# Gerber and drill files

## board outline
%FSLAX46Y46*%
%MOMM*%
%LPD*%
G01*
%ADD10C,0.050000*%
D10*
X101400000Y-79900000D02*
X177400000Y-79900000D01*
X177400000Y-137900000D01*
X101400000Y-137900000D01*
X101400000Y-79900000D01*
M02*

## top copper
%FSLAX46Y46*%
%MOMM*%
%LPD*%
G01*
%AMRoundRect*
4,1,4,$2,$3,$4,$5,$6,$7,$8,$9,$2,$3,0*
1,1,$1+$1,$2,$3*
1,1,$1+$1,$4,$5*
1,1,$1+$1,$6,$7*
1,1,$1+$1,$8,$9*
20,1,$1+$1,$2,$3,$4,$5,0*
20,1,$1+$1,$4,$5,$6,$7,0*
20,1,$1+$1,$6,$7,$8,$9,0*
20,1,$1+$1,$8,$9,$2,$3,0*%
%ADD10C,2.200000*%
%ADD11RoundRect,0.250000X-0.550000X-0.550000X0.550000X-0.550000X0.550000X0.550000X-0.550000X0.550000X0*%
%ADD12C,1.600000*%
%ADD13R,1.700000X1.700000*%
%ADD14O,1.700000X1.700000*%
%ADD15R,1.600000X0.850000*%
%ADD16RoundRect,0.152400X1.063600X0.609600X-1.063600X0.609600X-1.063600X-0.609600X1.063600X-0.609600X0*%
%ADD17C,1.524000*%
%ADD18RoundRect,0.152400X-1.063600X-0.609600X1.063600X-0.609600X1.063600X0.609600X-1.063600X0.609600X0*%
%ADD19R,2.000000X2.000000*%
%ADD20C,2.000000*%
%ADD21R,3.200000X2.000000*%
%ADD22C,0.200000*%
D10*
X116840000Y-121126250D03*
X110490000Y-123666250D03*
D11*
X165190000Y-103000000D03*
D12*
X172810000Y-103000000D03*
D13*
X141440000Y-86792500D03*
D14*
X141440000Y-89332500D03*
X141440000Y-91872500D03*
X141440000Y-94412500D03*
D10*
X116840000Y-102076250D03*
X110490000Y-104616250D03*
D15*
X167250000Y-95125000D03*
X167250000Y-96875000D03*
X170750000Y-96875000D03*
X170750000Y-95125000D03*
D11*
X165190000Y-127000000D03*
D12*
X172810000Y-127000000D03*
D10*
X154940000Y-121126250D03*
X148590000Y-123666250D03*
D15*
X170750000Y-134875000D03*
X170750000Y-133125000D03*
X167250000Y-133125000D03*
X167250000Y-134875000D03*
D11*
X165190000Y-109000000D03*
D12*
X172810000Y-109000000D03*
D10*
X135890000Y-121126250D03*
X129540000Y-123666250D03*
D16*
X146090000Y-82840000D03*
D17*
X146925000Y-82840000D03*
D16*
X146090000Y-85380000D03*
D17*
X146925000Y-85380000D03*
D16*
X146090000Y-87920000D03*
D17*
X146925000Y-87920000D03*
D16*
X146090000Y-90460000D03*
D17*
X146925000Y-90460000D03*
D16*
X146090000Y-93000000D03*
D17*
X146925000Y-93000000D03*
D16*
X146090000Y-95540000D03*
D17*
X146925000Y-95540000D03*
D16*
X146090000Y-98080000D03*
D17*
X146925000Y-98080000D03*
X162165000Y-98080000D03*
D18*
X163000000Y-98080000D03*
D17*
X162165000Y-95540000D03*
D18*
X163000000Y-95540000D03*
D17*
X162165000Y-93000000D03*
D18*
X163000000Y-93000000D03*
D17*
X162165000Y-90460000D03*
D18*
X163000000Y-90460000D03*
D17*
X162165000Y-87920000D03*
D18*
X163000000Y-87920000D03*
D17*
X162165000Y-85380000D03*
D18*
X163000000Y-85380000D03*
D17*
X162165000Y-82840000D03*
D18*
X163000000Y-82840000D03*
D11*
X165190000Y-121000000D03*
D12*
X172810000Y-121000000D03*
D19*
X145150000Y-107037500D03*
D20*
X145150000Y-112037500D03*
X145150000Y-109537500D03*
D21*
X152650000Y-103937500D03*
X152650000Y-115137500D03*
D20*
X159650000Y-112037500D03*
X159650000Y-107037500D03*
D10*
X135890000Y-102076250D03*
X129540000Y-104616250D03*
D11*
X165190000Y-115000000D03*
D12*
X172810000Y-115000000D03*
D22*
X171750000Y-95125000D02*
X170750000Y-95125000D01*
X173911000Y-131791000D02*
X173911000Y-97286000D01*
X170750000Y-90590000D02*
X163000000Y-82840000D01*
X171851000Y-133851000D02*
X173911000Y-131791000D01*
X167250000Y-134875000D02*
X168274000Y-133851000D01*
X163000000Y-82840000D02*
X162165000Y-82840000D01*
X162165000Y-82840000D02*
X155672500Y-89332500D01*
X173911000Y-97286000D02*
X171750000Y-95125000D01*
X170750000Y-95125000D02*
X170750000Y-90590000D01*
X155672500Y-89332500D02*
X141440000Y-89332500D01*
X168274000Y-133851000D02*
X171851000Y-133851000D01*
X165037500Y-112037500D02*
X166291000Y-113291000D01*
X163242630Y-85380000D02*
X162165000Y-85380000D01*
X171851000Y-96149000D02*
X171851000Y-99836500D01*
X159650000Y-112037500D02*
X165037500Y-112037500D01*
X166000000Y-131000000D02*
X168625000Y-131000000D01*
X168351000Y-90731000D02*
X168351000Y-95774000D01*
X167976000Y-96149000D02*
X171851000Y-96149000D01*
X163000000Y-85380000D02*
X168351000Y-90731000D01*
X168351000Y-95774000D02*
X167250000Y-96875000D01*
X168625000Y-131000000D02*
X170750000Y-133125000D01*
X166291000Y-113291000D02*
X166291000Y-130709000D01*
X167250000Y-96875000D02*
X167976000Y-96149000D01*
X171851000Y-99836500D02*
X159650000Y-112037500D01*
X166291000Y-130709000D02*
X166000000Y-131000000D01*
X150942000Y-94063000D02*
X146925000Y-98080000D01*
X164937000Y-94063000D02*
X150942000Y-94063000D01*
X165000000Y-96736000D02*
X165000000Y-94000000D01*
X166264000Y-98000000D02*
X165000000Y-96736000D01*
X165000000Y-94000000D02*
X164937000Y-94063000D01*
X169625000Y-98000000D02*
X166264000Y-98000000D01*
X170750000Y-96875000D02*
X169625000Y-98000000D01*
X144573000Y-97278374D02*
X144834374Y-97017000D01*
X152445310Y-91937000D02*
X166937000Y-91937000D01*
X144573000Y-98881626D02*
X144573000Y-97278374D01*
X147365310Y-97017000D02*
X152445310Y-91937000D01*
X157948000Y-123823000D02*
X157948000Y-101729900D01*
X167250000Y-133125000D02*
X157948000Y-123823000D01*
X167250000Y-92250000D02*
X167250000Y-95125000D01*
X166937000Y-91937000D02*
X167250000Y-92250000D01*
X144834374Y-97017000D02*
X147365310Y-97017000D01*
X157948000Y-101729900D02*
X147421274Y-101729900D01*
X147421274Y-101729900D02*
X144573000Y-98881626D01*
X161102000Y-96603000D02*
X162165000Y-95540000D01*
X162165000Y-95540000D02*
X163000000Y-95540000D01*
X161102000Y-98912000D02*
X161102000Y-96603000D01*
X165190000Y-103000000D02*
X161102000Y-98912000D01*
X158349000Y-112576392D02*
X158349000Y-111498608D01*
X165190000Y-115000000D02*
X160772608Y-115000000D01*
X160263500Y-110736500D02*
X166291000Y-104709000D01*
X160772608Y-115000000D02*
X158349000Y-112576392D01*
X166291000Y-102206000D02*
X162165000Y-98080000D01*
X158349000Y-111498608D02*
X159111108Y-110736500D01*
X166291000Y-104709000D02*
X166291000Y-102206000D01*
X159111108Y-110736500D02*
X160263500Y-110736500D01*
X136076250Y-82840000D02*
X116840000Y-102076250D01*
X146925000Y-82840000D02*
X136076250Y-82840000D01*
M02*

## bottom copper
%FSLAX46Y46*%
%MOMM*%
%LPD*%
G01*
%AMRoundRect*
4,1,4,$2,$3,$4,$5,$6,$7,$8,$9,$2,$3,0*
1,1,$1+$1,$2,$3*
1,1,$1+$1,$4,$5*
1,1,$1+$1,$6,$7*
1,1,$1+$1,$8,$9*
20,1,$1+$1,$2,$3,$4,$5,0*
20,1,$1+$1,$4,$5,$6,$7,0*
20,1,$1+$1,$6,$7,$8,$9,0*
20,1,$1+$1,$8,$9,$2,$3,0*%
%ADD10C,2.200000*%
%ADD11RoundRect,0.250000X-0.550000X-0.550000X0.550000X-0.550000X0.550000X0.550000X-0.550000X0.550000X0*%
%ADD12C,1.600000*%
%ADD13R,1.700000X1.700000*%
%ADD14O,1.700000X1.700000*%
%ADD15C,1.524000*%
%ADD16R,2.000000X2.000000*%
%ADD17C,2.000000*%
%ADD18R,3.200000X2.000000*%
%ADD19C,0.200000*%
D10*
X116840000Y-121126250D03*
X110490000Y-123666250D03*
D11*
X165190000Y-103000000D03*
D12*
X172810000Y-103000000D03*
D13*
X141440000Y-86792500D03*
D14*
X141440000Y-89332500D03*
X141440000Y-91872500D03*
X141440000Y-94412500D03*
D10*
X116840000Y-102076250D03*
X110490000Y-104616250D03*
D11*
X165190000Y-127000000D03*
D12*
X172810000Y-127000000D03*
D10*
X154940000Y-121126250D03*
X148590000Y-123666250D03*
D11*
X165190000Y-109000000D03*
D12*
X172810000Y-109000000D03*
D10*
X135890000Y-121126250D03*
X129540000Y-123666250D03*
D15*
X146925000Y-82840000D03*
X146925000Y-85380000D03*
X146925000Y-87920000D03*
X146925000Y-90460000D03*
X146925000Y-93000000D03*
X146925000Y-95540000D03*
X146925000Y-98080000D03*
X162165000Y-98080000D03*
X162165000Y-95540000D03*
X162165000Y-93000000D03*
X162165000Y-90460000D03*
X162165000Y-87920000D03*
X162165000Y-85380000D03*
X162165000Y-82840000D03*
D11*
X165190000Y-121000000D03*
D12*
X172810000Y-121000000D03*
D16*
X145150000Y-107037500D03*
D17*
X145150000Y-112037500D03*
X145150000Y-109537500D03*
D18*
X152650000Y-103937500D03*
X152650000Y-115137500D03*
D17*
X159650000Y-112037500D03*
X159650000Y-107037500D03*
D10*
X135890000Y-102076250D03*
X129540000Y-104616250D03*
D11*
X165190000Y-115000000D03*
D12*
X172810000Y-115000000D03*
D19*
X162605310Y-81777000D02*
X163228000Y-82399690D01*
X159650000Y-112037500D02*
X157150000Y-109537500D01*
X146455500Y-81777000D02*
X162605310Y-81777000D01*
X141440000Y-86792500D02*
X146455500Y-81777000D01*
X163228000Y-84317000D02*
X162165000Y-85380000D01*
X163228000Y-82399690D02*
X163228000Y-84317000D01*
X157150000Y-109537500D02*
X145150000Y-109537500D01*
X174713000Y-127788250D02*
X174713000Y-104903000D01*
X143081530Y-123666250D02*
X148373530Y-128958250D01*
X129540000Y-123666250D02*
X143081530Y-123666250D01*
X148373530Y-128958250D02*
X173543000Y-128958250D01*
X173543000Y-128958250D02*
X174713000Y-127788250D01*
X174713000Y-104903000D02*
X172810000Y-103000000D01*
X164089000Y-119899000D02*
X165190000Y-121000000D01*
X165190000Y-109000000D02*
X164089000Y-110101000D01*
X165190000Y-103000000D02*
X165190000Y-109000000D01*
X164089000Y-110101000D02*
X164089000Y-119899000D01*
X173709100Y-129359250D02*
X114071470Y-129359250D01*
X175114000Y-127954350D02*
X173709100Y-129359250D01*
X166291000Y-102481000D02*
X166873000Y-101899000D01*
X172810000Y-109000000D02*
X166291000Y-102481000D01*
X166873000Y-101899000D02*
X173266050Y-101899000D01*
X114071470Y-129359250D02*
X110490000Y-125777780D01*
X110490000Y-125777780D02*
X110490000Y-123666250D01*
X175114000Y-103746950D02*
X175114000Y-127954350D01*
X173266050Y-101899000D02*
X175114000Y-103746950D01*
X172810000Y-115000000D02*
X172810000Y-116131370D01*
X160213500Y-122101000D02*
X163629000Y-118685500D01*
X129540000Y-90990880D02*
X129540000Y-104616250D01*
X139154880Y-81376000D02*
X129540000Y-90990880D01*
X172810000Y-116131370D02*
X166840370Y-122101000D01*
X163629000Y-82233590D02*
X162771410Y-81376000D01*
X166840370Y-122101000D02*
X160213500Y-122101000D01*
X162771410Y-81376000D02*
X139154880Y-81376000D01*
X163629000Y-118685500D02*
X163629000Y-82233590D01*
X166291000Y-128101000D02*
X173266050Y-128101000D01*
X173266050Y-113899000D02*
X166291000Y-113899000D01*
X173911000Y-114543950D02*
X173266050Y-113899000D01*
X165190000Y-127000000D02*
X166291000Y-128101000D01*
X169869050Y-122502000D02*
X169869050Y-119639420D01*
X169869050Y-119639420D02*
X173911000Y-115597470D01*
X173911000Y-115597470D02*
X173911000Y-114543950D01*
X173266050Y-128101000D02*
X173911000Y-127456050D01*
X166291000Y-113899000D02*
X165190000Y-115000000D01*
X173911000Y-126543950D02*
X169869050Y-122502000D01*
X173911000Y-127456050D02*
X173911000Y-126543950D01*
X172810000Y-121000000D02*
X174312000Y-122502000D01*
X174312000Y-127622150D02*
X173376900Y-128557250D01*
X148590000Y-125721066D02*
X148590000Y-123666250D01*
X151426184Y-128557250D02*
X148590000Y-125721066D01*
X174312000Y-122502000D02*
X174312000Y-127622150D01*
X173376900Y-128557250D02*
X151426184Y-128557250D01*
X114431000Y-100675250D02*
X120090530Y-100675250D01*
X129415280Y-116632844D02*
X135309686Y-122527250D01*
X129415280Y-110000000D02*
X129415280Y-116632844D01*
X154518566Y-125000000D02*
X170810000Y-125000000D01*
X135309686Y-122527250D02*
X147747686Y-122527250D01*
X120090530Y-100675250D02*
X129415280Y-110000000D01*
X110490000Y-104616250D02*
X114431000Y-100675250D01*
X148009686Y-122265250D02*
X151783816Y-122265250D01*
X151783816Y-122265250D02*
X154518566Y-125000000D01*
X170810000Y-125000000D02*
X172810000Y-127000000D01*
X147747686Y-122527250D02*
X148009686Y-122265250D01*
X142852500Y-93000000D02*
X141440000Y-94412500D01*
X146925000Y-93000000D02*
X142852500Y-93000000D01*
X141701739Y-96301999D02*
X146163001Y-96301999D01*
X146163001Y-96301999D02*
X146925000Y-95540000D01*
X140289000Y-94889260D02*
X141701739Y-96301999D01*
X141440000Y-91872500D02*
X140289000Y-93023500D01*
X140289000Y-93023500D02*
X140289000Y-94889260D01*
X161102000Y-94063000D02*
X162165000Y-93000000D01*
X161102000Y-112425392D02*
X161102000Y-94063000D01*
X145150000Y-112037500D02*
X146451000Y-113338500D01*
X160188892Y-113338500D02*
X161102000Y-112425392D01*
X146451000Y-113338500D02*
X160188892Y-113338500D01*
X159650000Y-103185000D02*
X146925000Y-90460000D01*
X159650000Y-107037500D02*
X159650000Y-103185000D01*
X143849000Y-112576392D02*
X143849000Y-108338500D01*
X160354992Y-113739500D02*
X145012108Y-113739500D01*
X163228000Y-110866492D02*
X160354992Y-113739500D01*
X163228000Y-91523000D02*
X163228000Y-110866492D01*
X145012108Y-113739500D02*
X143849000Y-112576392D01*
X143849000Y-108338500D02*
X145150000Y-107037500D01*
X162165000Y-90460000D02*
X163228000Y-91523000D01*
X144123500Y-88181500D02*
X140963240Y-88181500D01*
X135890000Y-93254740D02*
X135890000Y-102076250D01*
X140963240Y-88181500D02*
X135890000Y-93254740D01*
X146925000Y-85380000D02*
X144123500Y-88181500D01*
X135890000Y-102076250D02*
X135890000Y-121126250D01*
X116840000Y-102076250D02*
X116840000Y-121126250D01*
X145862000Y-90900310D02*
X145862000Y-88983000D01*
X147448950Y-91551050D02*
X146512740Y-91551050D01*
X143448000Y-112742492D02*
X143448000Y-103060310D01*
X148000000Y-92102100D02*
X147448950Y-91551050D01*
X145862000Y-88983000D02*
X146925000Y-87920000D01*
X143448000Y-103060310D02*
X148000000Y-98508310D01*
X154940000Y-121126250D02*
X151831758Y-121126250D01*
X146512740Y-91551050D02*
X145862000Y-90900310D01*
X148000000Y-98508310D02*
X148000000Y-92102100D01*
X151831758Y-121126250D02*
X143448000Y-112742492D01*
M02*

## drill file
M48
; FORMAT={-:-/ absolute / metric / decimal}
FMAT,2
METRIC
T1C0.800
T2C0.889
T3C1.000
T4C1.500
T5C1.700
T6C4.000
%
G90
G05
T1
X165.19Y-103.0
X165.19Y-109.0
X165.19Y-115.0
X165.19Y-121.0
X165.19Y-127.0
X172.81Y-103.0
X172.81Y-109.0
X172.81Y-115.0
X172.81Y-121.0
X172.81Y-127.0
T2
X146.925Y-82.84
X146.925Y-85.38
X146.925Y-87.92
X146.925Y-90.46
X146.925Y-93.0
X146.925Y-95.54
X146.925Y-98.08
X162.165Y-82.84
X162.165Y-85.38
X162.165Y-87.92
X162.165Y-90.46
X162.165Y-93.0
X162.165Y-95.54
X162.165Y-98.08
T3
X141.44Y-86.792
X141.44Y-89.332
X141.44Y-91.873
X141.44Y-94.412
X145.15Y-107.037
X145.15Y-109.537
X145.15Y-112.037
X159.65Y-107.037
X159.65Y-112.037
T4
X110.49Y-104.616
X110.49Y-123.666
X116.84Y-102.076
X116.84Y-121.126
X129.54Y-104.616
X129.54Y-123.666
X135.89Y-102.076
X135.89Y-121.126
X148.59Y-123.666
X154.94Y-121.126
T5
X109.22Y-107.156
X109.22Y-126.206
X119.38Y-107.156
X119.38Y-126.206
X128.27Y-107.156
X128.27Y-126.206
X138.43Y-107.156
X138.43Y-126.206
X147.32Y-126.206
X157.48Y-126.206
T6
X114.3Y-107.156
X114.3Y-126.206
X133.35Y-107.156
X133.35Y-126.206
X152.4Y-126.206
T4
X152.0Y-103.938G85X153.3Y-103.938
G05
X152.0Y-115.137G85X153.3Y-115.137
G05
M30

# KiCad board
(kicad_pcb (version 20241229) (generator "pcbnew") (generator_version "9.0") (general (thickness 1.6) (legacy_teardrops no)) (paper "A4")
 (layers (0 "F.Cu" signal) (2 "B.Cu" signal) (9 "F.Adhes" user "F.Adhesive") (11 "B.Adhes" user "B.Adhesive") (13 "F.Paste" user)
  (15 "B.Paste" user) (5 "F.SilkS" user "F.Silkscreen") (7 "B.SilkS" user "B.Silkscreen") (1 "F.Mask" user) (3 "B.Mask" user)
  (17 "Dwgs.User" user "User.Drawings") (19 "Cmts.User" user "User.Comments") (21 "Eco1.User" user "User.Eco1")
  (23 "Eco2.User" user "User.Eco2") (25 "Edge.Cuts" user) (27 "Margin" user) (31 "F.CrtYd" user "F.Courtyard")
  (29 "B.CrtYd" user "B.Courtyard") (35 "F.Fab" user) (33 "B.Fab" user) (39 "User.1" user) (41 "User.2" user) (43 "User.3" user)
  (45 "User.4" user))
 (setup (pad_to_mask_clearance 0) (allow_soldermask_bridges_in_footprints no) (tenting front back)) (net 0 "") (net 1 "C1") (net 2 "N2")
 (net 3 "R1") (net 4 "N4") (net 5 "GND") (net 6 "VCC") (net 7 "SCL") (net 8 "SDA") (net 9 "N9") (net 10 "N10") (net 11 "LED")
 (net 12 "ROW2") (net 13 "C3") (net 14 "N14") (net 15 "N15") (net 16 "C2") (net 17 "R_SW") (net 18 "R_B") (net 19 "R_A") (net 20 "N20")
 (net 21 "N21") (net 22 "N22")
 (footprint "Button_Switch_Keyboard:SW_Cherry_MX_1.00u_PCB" (layer "F.Cu") (at 116.84 121.12625)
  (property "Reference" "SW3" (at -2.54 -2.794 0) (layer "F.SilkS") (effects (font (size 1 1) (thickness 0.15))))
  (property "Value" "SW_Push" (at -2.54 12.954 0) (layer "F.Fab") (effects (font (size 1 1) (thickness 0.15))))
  (pad "" np_thru_hole circle (at -7.62 5.08) (size 1.7 1.7) (drill 1.7) (layers "*.Cu" "*.Mask"))
  (pad "" np_thru_hole circle (at -2.54 5.08) (size 4 4) (drill 4) (layers "*.Cu" "*.Mask"))
  (pad "" np_thru_hole circle (at 2.54 5.08) (size 1.7 1.7) (drill 1.7) (layers "*.Cu" "*.Mask"))
  (pad "1" thru_hole circle (at 0 0) (size 2.2 2.2) (drill 1.5) (layers "*.Cu" "*.Mask") (remove_unused_layers no) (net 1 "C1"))
  (pad "2" thru_hole circle (at -6.35 2.54) (size 2.2 2.2) (drill 1.5) (layers "*.Cu" "*.Mask") (remove_unused_layers no) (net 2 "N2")))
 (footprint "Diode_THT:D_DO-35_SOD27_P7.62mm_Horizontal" (layer "F.Cu") (at 165.19 103)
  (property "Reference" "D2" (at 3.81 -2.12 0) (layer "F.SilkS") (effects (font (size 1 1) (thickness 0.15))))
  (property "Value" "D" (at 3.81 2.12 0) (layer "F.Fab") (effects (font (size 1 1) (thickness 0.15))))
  (pad "1" thru_hole roundrect (at 0 0) (size 1.6 1.6) (drill 0.8) (layers "*.Cu" "*.Mask") (remove_unused_layers no)
   (roundrect_rratio 0.15625) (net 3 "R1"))
  (pad "2" thru_hole circle (at 7.62 0) (size 1.6 1.6) (drill 0.8) (layers "*.Cu" "*.Mask") (remove_unused_layers no) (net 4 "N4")))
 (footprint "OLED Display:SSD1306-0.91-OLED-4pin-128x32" (layer "F.Cu") (at 104.94 84.6025)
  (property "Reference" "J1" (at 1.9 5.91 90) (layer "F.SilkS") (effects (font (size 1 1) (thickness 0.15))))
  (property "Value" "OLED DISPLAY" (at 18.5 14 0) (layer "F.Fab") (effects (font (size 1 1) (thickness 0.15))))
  (pad "1" thru_hole rect (at 36.5 2.19) (size 1.7 1.7) (drill 1) (layers "*.Cu" "*.Mask") (remove_unused_layers no) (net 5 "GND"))
  (pad "2" thru_hole oval (at 36.5 4.73) (size 1.7 1.7) (drill 1) (layers "*.Cu" "*.Mask") (remove_unused_layers no) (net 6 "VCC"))
  (pad "3" thru_hole oval (at 36.5 7.27) (size 1.7 1.7) (drill 1) (layers "*.Cu" "*.Mask") (remove_unused_layers no) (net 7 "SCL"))
  (pad "4" thru_hole oval (at 36.5 9.81) (size 1.7 1.7) (drill 1) (layers "*.Cu" "*.Mask") (remove_unused_layers no) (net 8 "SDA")))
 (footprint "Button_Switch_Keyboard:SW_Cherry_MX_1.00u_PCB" (layer "F.Cu") (at 116.84 102.07625)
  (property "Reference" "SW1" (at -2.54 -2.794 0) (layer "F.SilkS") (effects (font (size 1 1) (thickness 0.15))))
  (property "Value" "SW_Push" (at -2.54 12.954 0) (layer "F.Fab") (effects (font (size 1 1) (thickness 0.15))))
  (pad "" np_thru_hole circle (at -7.62 5.08) (size 1.7 1.7) (drill 1.7) (layers "*.Cu" "*.Mask"))
  (pad "" np_thru_hole circle (at -2.54 5.08) (size 4 4) (drill 4) (layers "*.Cu" "*.Mask"))
  (pad "" np_thru_hole circle (at 2.54 5.08) (size 1.7 1.7) (drill 1.7) (layers "*.Cu" "*.Mask"))
  (pad "1" thru_hole circle (at 0 0) (size 2.2 2.2) (drill 1.5) (layers "*.Cu" "*.Mask") (remove_unused_layers no) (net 1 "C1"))
  (pad "2" thru_hole circle (at -6.35 2.54) (size 2.2 2.2) (drill 1.5) (layers "*.Cu" "*.Mask") (remove_unused_layers no) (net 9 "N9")))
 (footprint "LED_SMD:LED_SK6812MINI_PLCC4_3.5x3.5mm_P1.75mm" (layer "F.Cu") (at 169 96)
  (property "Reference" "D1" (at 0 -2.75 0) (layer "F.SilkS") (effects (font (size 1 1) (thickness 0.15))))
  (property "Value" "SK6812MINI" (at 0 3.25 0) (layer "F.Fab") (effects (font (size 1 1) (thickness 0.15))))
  (pad "1" smd rect (at -1.75 -0.875) (size 1.6 0.85) (layers "F.Cu" "F.Mask" "F.Paste") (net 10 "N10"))
  (pad "2" smd rect (at -1.75 0.875) (size 1.6 0.85) (layers "F.Cu" "F.Mask" "F.Paste") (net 5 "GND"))
  (pad "3" smd rect (at 1.75 0.875) (size 1.6 0.85) (layers "F.Cu" "F.Mask" "F.Paste") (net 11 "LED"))
  (pad "4" smd rect (at 1.75 -0.875) (size 1.6 0.85) (layers "F.Cu" "F.Mask" "F.Paste") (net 6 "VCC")))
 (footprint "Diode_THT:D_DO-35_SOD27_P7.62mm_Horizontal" (layer "F.Cu") (at 165.19 127)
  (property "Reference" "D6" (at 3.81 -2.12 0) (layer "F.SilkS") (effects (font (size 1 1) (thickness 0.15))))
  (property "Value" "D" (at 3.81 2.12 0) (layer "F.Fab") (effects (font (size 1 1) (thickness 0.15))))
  (pad "1" thru_hole roundrect (at 0 0) (size 1.6 1.6) (drill 0.8) (layers "*.Cu" "*.Mask") (remove_unused_layers no)
   (roundrect_rratio 0.15625) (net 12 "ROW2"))
  (pad "2" thru_hole circle (at 7.62 0) (size 1.6 1.6) (drill 0.8) (layers "*.Cu" "*.Mask") (remove_unused_layers no) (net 9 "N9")))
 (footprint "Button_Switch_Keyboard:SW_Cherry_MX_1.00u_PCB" (layer "F.Cu") (at 154.94 121.12625)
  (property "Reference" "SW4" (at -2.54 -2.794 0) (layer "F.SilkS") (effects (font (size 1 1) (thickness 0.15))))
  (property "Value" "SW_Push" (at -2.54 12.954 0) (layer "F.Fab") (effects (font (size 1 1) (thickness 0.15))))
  (pad "" np_thru_hole circle (at -7.62 5.08) (size 1.7 1.7) (drill 1.7) (layers "*.Cu" "*.Mask"))
  (pad "" np_thru_hole circle (at -2.54 5.08) (size 4 4) (drill 4) (layers "*.Cu" "*.Mask"))
  (pad "" np_thru_hole circle (at 2.54 5.08) (size 1.7 1.7) (drill 1.7) (layers "*.Cu" "*.Mask"))
  (pad "1" thru_hole circle (at 0 0) (size 2.2 2.2) (drill 1.5) (layers "*.Cu" "*.Mask") (remove_unused_layers no) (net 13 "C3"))
  (pad "2" thru_hole circle (at -6.35 2.54) (size 2.2 2.2) (drill 1.5) (layers "*.Cu" "*.Mask") (remove_unused_layers no) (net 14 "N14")))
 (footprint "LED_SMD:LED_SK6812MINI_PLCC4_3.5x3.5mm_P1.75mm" (layer "F.Cu") (at 169 134 180)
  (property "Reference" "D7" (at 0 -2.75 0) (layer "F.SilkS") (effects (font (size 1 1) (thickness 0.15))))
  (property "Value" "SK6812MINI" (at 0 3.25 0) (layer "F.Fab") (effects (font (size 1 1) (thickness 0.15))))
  (pad "1" smd rect (at -1.75 -0.875 180) (size 1.6 0.85) (layers "F.Cu" "F.Mask" "F.Paste") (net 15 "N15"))
  (pad "2" smd rect (at -1.75 0.875 180) (size 1.6 0.85) (layers "F.Cu" "F.Mask" "F.Paste") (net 5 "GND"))
  (pad "3" smd rect (at 1.75 0.875 180) (size 1.6 0.85) (layers "F.Cu" "F.Mask" "F.Paste") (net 10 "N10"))
  (pad "4" smd rect (at 1.75 -0.875 180) (size 1.6 0.85) (layers "F.Cu" "F.Mask" "F.Paste") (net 6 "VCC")))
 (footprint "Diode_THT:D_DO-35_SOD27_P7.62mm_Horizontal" (layer "F.Cu") (at 165.19 109)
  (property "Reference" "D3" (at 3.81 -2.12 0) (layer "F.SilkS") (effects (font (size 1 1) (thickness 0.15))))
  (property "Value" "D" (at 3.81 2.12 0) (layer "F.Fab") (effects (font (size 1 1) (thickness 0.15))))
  (pad "1" thru_hole roundrect (at 0 0) (size 1.6 1.6) (drill 0.8) (layers "*.Cu" "*.Mask") (remove_unused_layers no)
   (roundrect_rratio 0.15625) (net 3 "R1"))
  (pad "2" thru_hole circle (at 7.62 0) (size 1.6 1.6) (drill 0.8) (layers "*.Cu" "*.Mask") (remove_unused_layers no) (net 2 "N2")))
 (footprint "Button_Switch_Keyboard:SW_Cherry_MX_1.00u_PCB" (layer "F.Cu") (at 135.89 121.12625)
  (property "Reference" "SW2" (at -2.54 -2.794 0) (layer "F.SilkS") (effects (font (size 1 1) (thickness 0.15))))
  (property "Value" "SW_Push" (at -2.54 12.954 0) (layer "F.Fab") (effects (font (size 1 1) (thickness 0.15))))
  (pad "" np_thru_hole circle (at -7.62 5.08) (size 1.7 1.7) (drill 1.7) (layers "*.Cu" "*.Mask"))
  (pad "" np_thru_hole circle (at -2.54 5.08) (size 4 4) (drill 4) (layers "*.Cu" "*.Mask"))
  (pad "" np_thru_hole circle (at 2.54 5.08) (size 1.7 1.7) (drill 1.7) (layers "*.Cu" "*.Mask"))
  (pad "1" thru_hole circle (at 0 0) (size 2.2 2.2) (drill 1.5) (layers "*.Cu" "*.Mask") (remove_unused_layers no) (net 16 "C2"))
  (pad "2" thru_hole circle (at -6.35 2.54) (size 2.2 2.2) (drill 1.5) (layers "*.Cu" "*.Mask") (remove_unused_layers no) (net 4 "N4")))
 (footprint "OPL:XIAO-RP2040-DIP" (layer "F.Cu") (at 154.545 90.46)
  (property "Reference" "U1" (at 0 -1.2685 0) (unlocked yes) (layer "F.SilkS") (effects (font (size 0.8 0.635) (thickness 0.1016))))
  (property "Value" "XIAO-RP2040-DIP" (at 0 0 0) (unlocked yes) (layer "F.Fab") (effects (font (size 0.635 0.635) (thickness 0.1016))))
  (pad "1" smd roundrect (at -8.455 -7.62 180) (size 2.432 1.524) (layers "F.Cu" "F.Mask") (roundrect_rratio 0.1) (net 1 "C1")
   (thermal_bridge_angle 45))
  (pad "1" thru_hole circle (at -7.62 -7.62 180) (size 1.524 1.524) (drill 0.889) (layers "*.Cu" "*.Mask") (remove_unused_layers no)
   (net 1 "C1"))
  (pad "2" smd roundrect (at -8.455 -5.08 180) (size 2.432 1.524) (layers "F.Cu" "F.Mask") (roundrect_rratio 0.1) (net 16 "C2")
   (thermal_bridge_angle 45))
  (pad "2" thru_hole circle (at -7.62 -5.08 180) (size 1.524 1.524) (drill 0.889) (layers "*.Cu" "*.Mask") (remove_unused_layers no)
   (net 16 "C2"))
  (pad "3" smd roundrect (at -8.455 -2.54 180) (size 2.432 1.524) (layers "F.Cu" "F.Mask") (roundrect_rratio 0.1) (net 13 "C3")
   (thermal_bridge_angle 45))
  (pad "3" thru_hole circle (at -7.62 -2.54 180) (size 1.524 1.524) (drill 0.889) (layers "*.Cu" "*.Mask") (remove_unused_layers no)
   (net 13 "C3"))
  (pad "4" smd roundrect (at -8.455 0 180) (size 2.432 1.524) (layers "F.Cu" "F.Mask") (roundrect_rratio 0.1) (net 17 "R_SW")
   (thermal_bridge_angle 45))
  (pad "4" thru_hole circle (at -7.62 0 180) (size 1.524 1.524) (drill 0.889) (layers "*.Cu" "*.Mask") (remove_unused_layers no)
   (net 17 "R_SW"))
  (pad "5" smd roundrect (at -8.455 2.54 180) (size 2.432 1.524) (layers "F.Cu" "F.Mask") (roundrect_rratio 0.1) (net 8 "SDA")
   (thermal_bridge_angle 45))
  (pad "5" thru_hole circle (at -7.62 2.54 180) (size 1.524 1.524) (drill 0.889) (layers "*.Cu" "*.Mask") (remove_unused_layers no)
   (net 8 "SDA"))
  (pad "6" smd roundrect (at -8.455 5.08 180) (size 2.432 1.524) (layers "F.Cu" "F.Mask") (roundrect_rratio 0.1) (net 7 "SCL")
   (thermal_bridge_angle 45))
  (pad "6" thru_hole circle (at -7.62 5.08 180) (size 1.524 1.524) (drill 0.889) (layers "*.Cu" "*.Mask") (remove_unused_layers no)
   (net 7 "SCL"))
  (pad "7" smd roundrect (at -8.455 7.62 180) (size 2.432 1.524) (layers "F.Cu" "F.Mask") (roundrect_rratio 0.1) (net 11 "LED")
   (thermal_bridge_angle 45))
  (pad "7" thru_hole circle (at -7.62 7.62 180) (size 1.524 1.524) (drill 0.889) (layers "*.Cu" "*.Mask") (remove_unused_layers no)
   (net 11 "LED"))
  (pad "8" thru_hole circle (at 7.62 7.62) (size 1.524 1.524) (drill 0.889) (layers "*.Cu" "*.Mask") (remove_unused_layers no)
   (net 12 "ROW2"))
  (pad "8" smd roundrect (at 8.455 7.62) (size 2.432 1.524) (layers "F.Cu" "F.Mask") (roundrect_rratio 0.1) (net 12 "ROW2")
   (thermal_bridge_angle 45))
  (pad "9" thru_hole circle (at 7.62 5.08) (size 1.524 1.524) (drill 0.889) (layers "*.Cu" "*.Mask") (remove_unused_layers no) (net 3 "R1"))
  (pad "9" smd roundrect (at 8.455 5.08) (size 2.432 1.524) (layers "F.Cu" "F.Mask") (roundrect_rratio 0.1) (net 3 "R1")
   (thermal_bridge_angle 45))
  (pad "10" thru_hole circle (at 7.62 2.54) (size 1.524 1.524) (drill 0.889) (layers "*.Cu" "*.Mask") (remove_unused_layers no)
   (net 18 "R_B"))
  (pad "10" smd roundrect (at 8.455 2.54) (size 2.432 1.524) (layers "F.Cu" "F.Mask") (roundrect_rratio 0.1) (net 18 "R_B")
   (thermal_bridge_angle 45))
  (pad "11" thru_hole circle (at 7.62 0) (size 1.524 1.524) (drill 0.889) (layers "*.Cu" "*.Mask") (remove_unused_layers no) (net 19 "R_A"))
  (pad "11" smd roundrect (at 8.455 0) (size 2.432 1.524) (layers "F.Cu" "F.Mask") (roundrect_rratio 0.1) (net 19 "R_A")
   (thermal_bridge_angle 45))
  (pad "12" thru_hole circle (at 7.62 -2.54) (size 1.524 1.524) (drill 0.889) (layers "*.Cu" "*.Mask") (remove_unused_layers no)
   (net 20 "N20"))
  (pad "12" smd roundrect (at 8.455 -2.54) (size 2.432 1.524) (layers "F.Cu" "F.Mask") (roundrect_rratio 0.1) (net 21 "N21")
   (thermal_bridge_angle 45))
  (pad "13" thru_hole circle (at 7.62 -5.08) (size 1.524 1.524) (drill 0.889) (layers "*.Cu" "*.Mask") (remove_unused_layers no)
   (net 5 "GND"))
  (pad "13" smd roundrect (at 8.455 -5.08) (size 2.432 1.524) (layers "F.Cu" "F.Mask") (roundrect_rratio 0.1) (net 5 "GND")
   (thermal_bridge_angle 45))
  (pad "14" thru_hole circle (at 7.62 -7.62) (size 1.524 1.524) (drill 0.889) (layers "*.Cu" "*.Mask") (remove_unused_layers no)
   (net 6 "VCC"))
  (pad "14" smd roundrect (at 8.455 -7.62) (size 2.432 1.524) (layers "F.Cu" "F.Mask") (roundrect_rratio 0.1) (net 6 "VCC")
   (thermal_bridge_angle 45)))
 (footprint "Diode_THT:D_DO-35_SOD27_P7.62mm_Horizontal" (layer "F.Cu") (at 165.19 121)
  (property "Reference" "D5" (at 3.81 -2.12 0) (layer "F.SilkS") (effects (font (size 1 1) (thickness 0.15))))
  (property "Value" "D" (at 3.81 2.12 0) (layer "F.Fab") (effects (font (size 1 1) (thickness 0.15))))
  (pad "1" thru_hole roundrect (at 0 0) (size 1.6 1.6) (drill 0.8) (layers "*.Cu" "*.Mask") (remove_unused_layers no)
   (roundrect_rratio 0.15625) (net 3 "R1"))
  (pad "2" thru_hole circle (at 7.62 0) (size 1.6 1.6) (drill 0.8) (layers "*.Cu" "*.Mask") (remove_unused_layers no) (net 14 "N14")))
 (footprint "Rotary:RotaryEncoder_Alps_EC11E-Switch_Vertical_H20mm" (layer "F.Cu") (at 145.15 107.0375)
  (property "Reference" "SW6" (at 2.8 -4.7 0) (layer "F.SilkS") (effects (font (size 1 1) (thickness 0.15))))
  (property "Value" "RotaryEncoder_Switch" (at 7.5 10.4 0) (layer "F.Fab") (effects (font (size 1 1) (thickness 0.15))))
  (pad "A" thru_hole rect (at 0 0) (size 2 2) (drill 1) (layers "*.Cu" "*.Mask") (remove_unused_layers no) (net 19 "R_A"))
  (pad "B" thru_hole circle (at 0 5) (size 2 2) (drill 1) (layers "*.Cu" "*.Mask") (remove_unused_layers no) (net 18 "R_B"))
  (pad "C" thru_hole circle (at 0 2.5) (size 2 2) (drill 1) (layers "*.Cu" "*.Mask") (remove_unused_layers no) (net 5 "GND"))
  (pad "MP" thru_hole rect (at 7.5 -3.1) (size 3.2 2) (drill oval 2.8 1.5) (layers "*.Cu" "*.Mask") (remove_unused_layers no))
  (pad "MP" thru_hole rect (at 7.5 8.1) (size 3.2 2) (drill oval 2.8 1.5) (layers "*.Cu" "*.Mask") (remove_unused_layers no))
  (pad "S1" thru_hole circle (at 14.5 5) (size 2 2) (drill 1) (layers "*.Cu" "*.Mask") (remove_unused_layers no) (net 5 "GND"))
  (pad "S2" thru_hole circle (at 14.5 0) (size 2 2) (drill 1) (layers "*.Cu" "*.Mask") (remove_unused_layers no) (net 17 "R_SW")))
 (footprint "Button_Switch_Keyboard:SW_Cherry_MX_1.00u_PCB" (layer "F.Cu") (at 135.89 102.07625)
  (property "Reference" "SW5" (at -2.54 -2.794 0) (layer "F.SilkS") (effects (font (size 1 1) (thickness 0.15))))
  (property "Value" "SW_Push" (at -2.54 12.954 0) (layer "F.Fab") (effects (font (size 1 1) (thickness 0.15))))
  (pad "" np_thru_hole circle (at -7.62 5.08) (size 1.7 1.7) (drill 1.7) (layers "*.Cu" "*.Mask"))
  (pad "" np_thru_hole circle (at -2.54 5.08) (size 4 4) (drill 4) (layers "*.Cu" "*.Mask"))
  (pad "" np_thru_hole circle (at 2.54 5.08) (size 1.7 1.7) (drill 1.7) (layers "*.Cu" "*.Mask"))
  (pad "1" thru_hole circle (at 0 0) (size 2.2 2.2) (drill 1.5) (layers "*.Cu" "*.Mask") (remove_unused_layers no) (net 16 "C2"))
  (pad "2" thru_hole circle (at -6.35 2.54) (size 2.2 2.2) (drill 1.5) (layers "*.Cu" "*.Mask") (remove_unused_layers no) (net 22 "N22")))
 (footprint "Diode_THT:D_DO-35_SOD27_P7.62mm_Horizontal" (layer "F.Cu") (at 165.19 115)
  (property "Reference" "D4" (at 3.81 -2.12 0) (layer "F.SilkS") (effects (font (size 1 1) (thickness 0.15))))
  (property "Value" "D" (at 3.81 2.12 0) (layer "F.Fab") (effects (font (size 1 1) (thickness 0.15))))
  (pad "1" thru_hole roundrect (at 0 0) (size 1.6 1.6) (drill 0.8) (layers "*.Cu" "*.Mask") (remove_unused_layers no)
   (roundrect_rratio 0.15625) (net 12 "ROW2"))
  (pad "2" thru_hole circle (at 7.62 0) (size 1.6 1.6) (drill 0.8) (layers "*.Cu" "*.Mask") (remove_unused_layers no) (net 22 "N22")))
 (gr_rect (start 101.4 79.9) (end 177.4 137.9) (stroke (width 0.05) (type default)) (fill no) (layer "Edge.Cuts"))
 (segment (start 171.75 95.125) (end 170.75 95.125) (width 0.2) (layer "F.Cu") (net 6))
 (segment (start 173.911 131.791) (end 173.911 97.286) (width 0.2) (layer "F.Cu") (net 6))
 (segment (start 170.75 90.59) (end 163 82.84) (width 0.2) (layer "F.Cu") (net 6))
 (segment (start 171.851 133.851) (end 173.911 131.791) (width 0.2) (layer "F.Cu") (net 6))
 (segment (start 167.25 134.875) (end 168.274 133.851) (width 0.2) (layer "F.Cu") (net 6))
 (segment (start 163 82.84) (end 162.165 82.84) (width 0.2) (layer "F.Cu") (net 6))
 (segment (start 162.165 82.84) (end 155.6725 89.3325) (width 0.2) (layer "F.Cu") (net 6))
 (segment (start 173.911 97.286) (end 171.75 95.125) (width 0.2) (layer "F.Cu") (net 6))
 (segment (start 170.75 95.125) (end 170.75 90.59) (width 0.2) (layer "F.Cu") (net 6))
 (segment (start 155.6725 89.3325) (end 141.44 89.3325) (width 0.2) (layer "F.Cu") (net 6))
 (segment (start 168.274 133.851) (end 171.851 133.851) (width 0.2) (layer "F.Cu") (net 6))
 (segment (start 165.0375 112.0375) (end 166.291 113.291) (width 0.2) (layer "F.Cu") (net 5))
 (segment (start 163.24263 85.38) (end 162.165 85.38) (width 0.2) (layer "F.Cu") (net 5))
 (segment (start 171.851 96.149) (end 171.851 99.8365) (width 0.2) (layer "F.Cu") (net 5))
 (segment (start 159.65 112.0375) (end 165.0375 112.0375) (width 0.2) (layer "F.Cu") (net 5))
 (segment (start 166 131) (end 168.625 131) (width 0.2) (layer "F.Cu") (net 5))
 (segment (start 168.351 90.731) (end 168.351 95.774) (width 0.2) (layer "F.Cu") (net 5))
 (segment (start 167.976 96.149) (end 171.851 96.149) (width 0.2) (layer "F.Cu") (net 5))
 (segment (start 163 85.38) (end 168.351 90.731) (width 0.2) (layer "F.Cu") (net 5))
 (segment (start 168.351 95.774) (end 167.25 96.875) (width 0.2) (layer "F.Cu") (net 5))
 (segment (start 168.625 131) (end 170.75 133.125) (width 0.2) (layer "F.Cu") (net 5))
 (segment (start 166.291 113.291) (end 166.291 130.709) (width 0.2) (layer "F.Cu") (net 5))
 (segment (start 167.25 96.875) (end 167.976 96.149) (width 0.2) (layer "F.Cu") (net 5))
 (segment (start 171.851 99.8365) (end 159.65 112.0375) (width 0.2) (layer "F.Cu") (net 5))
 (segment (start 166.291 130.709) (end 166 131) (width 0.2) (layer "F.Cu") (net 5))
 (segment (start 162.60531 81.777) (end 163.228 82.39969) (width 0.2) (layer "B.Cu") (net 5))
 (segment (start 159.65 112.0375) (end 157.15 109.5375) (width 0.2) (layer "B.Cu") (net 5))
 (segment (start 146.4555 81.777) (end 162.60531 81.777) (width 0.2) (layer "B.Cu") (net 5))
 (segment (start 141.44 86.7925) (end 146.4555 81.777) (width 0.2) (layer "B.Cu") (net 5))
 (segment (start 163.228 84.317) (end 162.165 85.38) (width 0.2) (layer "B.Cu") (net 5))
 (segment (start 163.228 82.39969) (end 163.228 84.317) (width 0.2) (layer "B.Cu") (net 5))
 (segment (start 157.15 109.5375) (end 145.15 109.5375) (width 0.2) (layer "B.Cu") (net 5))
 (segment (start 150.942 94.063) (end 146.925 98.08) (width 0.2) (layer "F.Cu") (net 11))
 (segment (start 164.937 94.063) (end 150.942 94.063) (width 0.2) (layer "F.Cu") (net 11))
 (segment (start 165 96.736) (end 165 94) (width 0.2) (layer "F.Cu") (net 11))
 (segment (start 166.264 98) (end 165 96.736) (width 0.2) (layer "F.Cu") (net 11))
 (segment (start 165 94) (end 164.937 94.063) (width 0.2) (layer "F.Cu") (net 11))
 (segment (start 169.625 98) (end 166.264 98) (width 0.2) (layer "F.Cu") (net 11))
 (segment (start 170.75 96.875) (end 169.625 98) (width 0.2) (layer "F.Cu") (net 11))
 (segment (start 144.573 97.278374) (end 144.834374 97.017) (width 0.2) (layer "F.Cu") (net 10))
 (segment (start 152.44531 91.937) (end 166.937 91.937) (width 0.2) (layer "F.Cu") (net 10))
 (segment (start 144.573 98.881626) (end 144.573 97.278374) (width 0.2) (layer "F.Cu") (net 10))
 (segment (start 147.36531 97.017) (end 152.44531 91.937) (width 0.2) (layer "F.Cu") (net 10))
 (segment (start 157.948 123.823) (end 157.948 101.7299) (width 0.2) (layer "F.Cu") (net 10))
 (segment (start 167.25 133.125) (end 157.948 123.823) (width 0.2) (layer "F.Cu") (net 10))
 (segment (start 167.25 92.25) (end 167.25 95.125) (width 0.2) (layer "F.Cu") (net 10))
 (segment (start 166.937 91.937) (end 167.25 92.25) (width 0.2) (layer "F.Cu") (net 10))
 (segment (start 144.834374 97.017) (end 147.36531 97.017) (width 0.2) (layer "F.Cu") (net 10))
 (segment (start 157.948 101.7299) (end 147.421274 101.7299) (width 0.2) (layer "F.Cu") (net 10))
 (segment (start 147.421274 101.7299) (end 144.573 98.881626) (width 0.2) (layer "F.Cu") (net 10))
 (segment (start 174.713 127.78825) (end 174.713 104.903) (width 0.2) (layer "B.Cu") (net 4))
 (segment (start 143.08153 123.66625) (end 148.37353 128.95825) (width 0.2) (layer "B.Cu") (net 4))
 (segment (start 129.54 123.66625) (end 143.08153 123.66625) (width 0.2) (layer "B.Cu") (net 4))
 (segment (start 148.37353 128.95825) (end 173.543 128.95825) (width 0.2) (layer "B.Cu") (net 4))
 (segment (start 173.543 128.95825) (end 174.713 127.78825) (width 0.2) (layer "B.Cu") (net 4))
 (segment (start 174.713 104.903) (end 172.81 103) (width 0.2) (layer "B.Cu") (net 4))
 (segment (start 161.102 96.603) (end 162.165 95.54) (width 0.2) (layer "F.Cu") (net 3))
 (segment (start 162.165 95.54) (end 163 95.54) (width 0.2) (layer "F.Cu") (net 3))
 (segment (start 161.102 98.912) (end 161.102 96.603) (width 0.2) (layer "F.Cu") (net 3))
 (segment (start 165.19 103) (end 161.102 98.912) (width 0.2) (layer "F.Cu") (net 3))
 (segment (start 164.089 119.899) (end 165.19 121) (width 0.2) (layer "B.Cu") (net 3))
 (segment (start 165.19 109) (end 164.089 110.101) (width 0.2) (layer "B.Cu") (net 3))
 (segment (start 165.19 103) (end 165.19 109) (width 0.2) (layer "B.Cu") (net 3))
 (segment (start 164.089 110.101) (end 164.089 119.899) (width 0.2) (layer "B.Cu") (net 3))
 (segment (start 173.7091 129.35925) (end 114.07147 129.35925) (width 0.2) (layer "B.Cu") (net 2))
 (segment (start 175.114 127.95435) (end 173.7091 129.35925) (width 0.2) (layer "B.Cu") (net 2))
 (segment (start 166.291 102.481) (end 166.873 101.899) (width 0.2) (layer "B.Cu") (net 2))
 (segment (start 172.81 109) (end 166.291 102.481) (width 0.2) (layer "B.Cu") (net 2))
 (segment (start 166.873 101.899) (end 173.26605 101.899) (width 0.2) (layer "B.Cu") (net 2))
 (segment (start 114.07147 129.35925) (end 110.49 125.77778) (width 0.2) (layer "B.Cu") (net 2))
 (segment (start 110.49 125.77778) (end 110.49 123.66625) (width 0.2) (layer "B.Cu") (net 2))
 (segment (start 175.114 103.74695) (end 175.114 127.95435) (width 0.2) (layer "B.Cu") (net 2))
 (segment (start 173.26605 101.899) (end 175.114 103.74695) (width 0.2) (layer "B.Cu") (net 2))
 (segment (start 172.81 115) (end 172.81 116.13137) (width 0.2) (layer "B.Cu") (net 22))
 (segment (start 160.2135 122.101) (end 163.629 118.6855) (width 0.2) (layer "B.Cu") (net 22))
 (segment (start 129.54 90.99088) (end 129.54 104.61625) (width 0.2) (layer "B.Cu") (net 22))
 (segment (start 139.15488 81.376) (end 129.54 90.99088) (width 0.2) (layer "B.Cu") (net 22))
 (segment (start 172.81 116.13137) (end 166.84037 122.101) (width 0.2) (layer "B.Cu") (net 22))
 (segment (start 163.629 82.23359) (end 162.77141 81.376) (width 0.2) (layer "B.Cu") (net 22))
 (segment (start 166.84037 122.101) (end 160.2135 122.101) (width 0.2) (layer "B.Cu") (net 22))
 (segment (start 162.77141 81.376) (end 139.15488 81.376) (width 0.2) (layer "B.Cu") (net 22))
 (segment (start 163.629 118.6855) (end 163.629 82.23359) (width 0.2) (layer "B.Cu") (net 22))
 (segment (start 158.349 112.576392) (end 158.349 111.498608) (width 0.2) (layer "F.Cu") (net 12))
 (segment (start 165.19 115) (end 160.772608 115) (width 0.2) (layer "F.Cu") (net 12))
 (segment (start 160.2635 110.7365) (end 166.291 104.709) (width 0.2) (layer "F.Cu") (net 12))
 (segment (start 160.772608 115) (end 158.349 112.576392) (width 0.2) (layer "F.Cu") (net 12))
 (segment (start 166.291 102.206) (end 162.165 98.08) (width 0.2) (layer "F.Cu") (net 12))
 (segment (start 158.349 111.498608) (end 159.111108 110.7365) (width 0.2) (layer "F.Cu") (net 12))
 (segment (start 166.291 104.709) (end 166.291 102.206) (width 0.2) (layer "F.Cu") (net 12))
 (segment (start 159.111108 110.7365) (end 160.2635 110.7365) (width 0.2) (layer "F.Cu") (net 12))
 (segment (start 166.291 128.101) (end 173.26605 128.101) (width 0.2) (layer "B.Cu") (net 12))
 (segment (start 173.26605 113.899) (end 166.291 113.899) (width 0.2) (layer "B.Cu") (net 12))
 (segment (start 173.911 114.54395) (end 173.26605 113.899) (width 0.2) (layer "B.Cu") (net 12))
 (segment (start 165.19 127) (end 166.291 128.101) (width 0.2) (layer "B.Cu") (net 12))
 (segment (start 169.86905 122.502) (end 169.86905 119.63942) (width 0.2) (layer "B.Cu") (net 12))
 (segment (start 169.86905 119.63942) (end 173.911 115.59747) (width 0.2) (layer "B.Cu") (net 12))
 (segment (start 173.911 115.59747) (end 173.911 114.54395) (width 0.2) (layer "B.Cu") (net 12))
 (segment (start 173.26605 128.101) (end 173.911 127.45605) (width 0.2) (layer "B.Cu") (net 12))
 (segment (start 166.291 113.899) (end 165.19 115) (width 0.2) (layer "B.Cu") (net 12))
 (segment (start 173.911 126.54395) (end 169.86905 122.502) (width 0.2) (layer "B.Cu") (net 12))
 (segment (start 173.911 127.45605) (end 173.911 126.54395) (width 0.2) (layer "B.Cu") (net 12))
 (segment (start 172.81 121) (end 174.312 122.502) (width 0.2) (layer "B.Cu") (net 14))
 (segment (start 174.312 127.62215) (end 173.3769 128.55725) (width 0.2) (layer "B.Cu") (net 14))
 (segment (start 148.59 125.721066) (end 148.59 123.66625) (width 0.2) (layer "B.Cu") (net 14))
 (segment (start 151.426184 128.55725) (end 148.59 125.721066) (width 0.2) (layer "B.Cu") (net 14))
 (segment (start 174.312 122.502) (end 174.312 127.62215) (width 0.2) (layer "B.Cu") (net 14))
 (segment (start 173.3769 128.55725) (end 151.426184 128.55725) (width 0.2) (layer "B.Cu") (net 14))
 (segment (start 114.431 100.67525) (end 120.09053 100.67525) (width 0.2) (layer "B.Cu") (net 9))
 (segment (start 129.41528 116.632844) (end 135.309686 122.52725) (width 0.2) (layer "B.Cu") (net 9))
 (segment (start 129.41528 110) (end 129.41528 116.632844) (width 0.2) (layer "B.Cu") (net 9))
 (segment (start 154.518566 125) (end 170.81 125) (width 0.2) (layer "B.Cu") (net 9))
 (segment (start 135.309686 122.52725) (end 147.747686 122.52725) (width 0.2) (layer "B.Cu") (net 9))
 (segment (start 120.09053 100.67525) (end 129.41528 110) (width 0.2) (layer "B.Cu") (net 9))
 (segment (start 110.49 104.61625) (end 114.431 100.67525) (width 0.2) (layer "B.Cu") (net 9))
 (segment (start 148.009686 122.26525) (end 151.783816 122.26525) (width 0.2) (layer "B.Cu") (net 9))
 (segment (start 151.783816 122.26525) (end 154.518566 125) (width 0.2) (layer "B.Cu") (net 9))
 (segment (start 170.81 125) (end 172.81 127) (width 0.2) (layer "B.Cu") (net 9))
 (segment (start 147.747686 122.52725) (end 148.009686 122.26525) (width 0.2) (layer "B.Cu") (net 9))
 (segment (start 142.8525 93) (end 141.44 94.4125) (width 0.2) (layer "B.Cu") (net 8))
 (segment (start 146.925 93) (end 142.8525 93) (width 0.2) (layer "B.Cu") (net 8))
 (segment (start 141.701739 96.301999) (end 146.163001 96.301999) (width 0.2) (layer "B.Cu") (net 7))
 (segment (start 146.163001 96.301999) (end 146.925 95.54) (width 0.2) (layer "B.Cu") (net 7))
 (segment (start 140.289 94.88926) (end 141.701739 96.301999) (width 0.2) (layer "B.Cu") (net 7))
 (segment (start 141.44 91.8725) (end 140.289 93.0235) (width 0.2) (layer "B.Cu") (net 7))
 (segment (start 140.289 93.0235) (end 140.289 94.88926) (width 0.2) (layer "B.Cu") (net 7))
 (segment (start 161.102 94.063) (end 162.165 93) (width 0.2) (layer "B.Cu") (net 18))
 (segment (start 161.102 112.425392) (end 161.102 94.063) (width 0.2) (layer "B.Cu") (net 18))
 (segment (start 145.15 112.0375) (end 146.451 113.3385) (width 0.2) (layer "B.Cu") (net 18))
 (segment (start 160.188892 113.3385) (end 161.102 112.425392) (width 0.2) (layer "B.Cu") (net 18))
 (segment (start 146.451 113.3385) (end 160.188892 113.3385) (width 0.2) (layer "B.Cu") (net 18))
 (segment (start 159.65 103.185) (end 146.925 90.46) (width 0.2) (layer "B.Cu") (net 17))
 (segment (start 159.65 107.0375) (end 159.65 103.185) (width 0.2) (layer "B.Cu") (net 17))
 (segment (start 143.849 112.576392) (end 143.849 108.3385) (width 0.2) (layer "B.Cu") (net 19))
 (segment (start 160.354992 113.7395) (end 145.012108 113.7395) (width 0.2) (layer "B.Cu") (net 19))
 (segment (start 163.228 110.866492) (end 160.354992 113.7395) (width 0.2) (layer "B.Cu") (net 19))
 (segment (start 163.228 91.523) (end 163.228 110.866492) (width 0.2) (layer "B.Cu") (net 19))
 (segment (start 145.012108 113.7395) (end 143.849 112.576392) (width 0.2) (layer "B.Cu") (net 19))
 (segment (start 143.849 108.3385) (end 145.15 107.0375) (width 0.2) (layer "B.Cu") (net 19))
 (segment (start 162.165 90.46) (end 163.228 91.523) (width 0.2) (layer "B.Cu") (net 19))
 (segment (start 144.1235 88.1815) (end 140.96324 88.1815) (width 0.2) (layer "B.Cu") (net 16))
 (segment (start 135.89 93.25474) (end 135.89 102.07625) (width 0.2) (layer "B.Cu") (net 16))
 (segment (start 140.96324 88.1815) (end 135.89 93.25474) (width 0.2) (layer "B.Cu") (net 16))
 (segment (start 146.925 85.38) (end 144.1235 88.1815) (width 0.2) (layer "B.Cu") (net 16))
 (segment (start 135.89 102.07625) (end 135.89 121.12625) (width 0.2) (layer "B.Cu") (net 16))
 (segment (start 136.07625 82.84) (end 116.84 102.07625) (width 0.2) (layer "F.Cu") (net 1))
 (segment (start 146.925 82.84) (end 136.07625 82.84) (width 0.2) (layer "F.Cu") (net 1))
 (segment (start 116.84 102.07625) (end 116.84 121.12625) (width 0.2) (layer "B.Cu") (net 1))
 (segment (start 145.862 90.90031) (end 145.862 88.983) (width 0.2) (layer "B.Cu") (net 13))
 (segment (start 147.44895 91.55105) (end 146.51274 91.55105) (width 0.2) (layer "B.Cu") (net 13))
 (segment (start 143.448 112.742492) (end 143.448 103.06031) (width 0.2) (layer "B.Cu") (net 13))
 (segment (start 148 92.1021) (end 147.44895 91.55105) (width 0.2) (layer "B.Cu") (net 13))
 (segment (start 145.862 88.983) (end 146.925 87.92) (width 0.2) (layer "B.Cu") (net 13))
 (segment (start 143.448 103.06031) (end 148 98.50831) (width 0.2) (layer "B.Cu") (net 13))
 (segment (start 154.94 121.12625) (end 151.831758 121.12625) (width 0.2) (layer "B.Cu") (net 13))
 (segment (start 146.51274 91.55105) (end 145.862 90.90031) (width 0.2) (layer "B.Cu") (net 13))
 (segment (start 148 98.50831) (end 148 92.1021) (width 0.2) (layer "B.Cu") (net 13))
 (segment (start 151.831758 121.12625) (end 143.448 112.742492) (width 0.2) (layer "B.Cu") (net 13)))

